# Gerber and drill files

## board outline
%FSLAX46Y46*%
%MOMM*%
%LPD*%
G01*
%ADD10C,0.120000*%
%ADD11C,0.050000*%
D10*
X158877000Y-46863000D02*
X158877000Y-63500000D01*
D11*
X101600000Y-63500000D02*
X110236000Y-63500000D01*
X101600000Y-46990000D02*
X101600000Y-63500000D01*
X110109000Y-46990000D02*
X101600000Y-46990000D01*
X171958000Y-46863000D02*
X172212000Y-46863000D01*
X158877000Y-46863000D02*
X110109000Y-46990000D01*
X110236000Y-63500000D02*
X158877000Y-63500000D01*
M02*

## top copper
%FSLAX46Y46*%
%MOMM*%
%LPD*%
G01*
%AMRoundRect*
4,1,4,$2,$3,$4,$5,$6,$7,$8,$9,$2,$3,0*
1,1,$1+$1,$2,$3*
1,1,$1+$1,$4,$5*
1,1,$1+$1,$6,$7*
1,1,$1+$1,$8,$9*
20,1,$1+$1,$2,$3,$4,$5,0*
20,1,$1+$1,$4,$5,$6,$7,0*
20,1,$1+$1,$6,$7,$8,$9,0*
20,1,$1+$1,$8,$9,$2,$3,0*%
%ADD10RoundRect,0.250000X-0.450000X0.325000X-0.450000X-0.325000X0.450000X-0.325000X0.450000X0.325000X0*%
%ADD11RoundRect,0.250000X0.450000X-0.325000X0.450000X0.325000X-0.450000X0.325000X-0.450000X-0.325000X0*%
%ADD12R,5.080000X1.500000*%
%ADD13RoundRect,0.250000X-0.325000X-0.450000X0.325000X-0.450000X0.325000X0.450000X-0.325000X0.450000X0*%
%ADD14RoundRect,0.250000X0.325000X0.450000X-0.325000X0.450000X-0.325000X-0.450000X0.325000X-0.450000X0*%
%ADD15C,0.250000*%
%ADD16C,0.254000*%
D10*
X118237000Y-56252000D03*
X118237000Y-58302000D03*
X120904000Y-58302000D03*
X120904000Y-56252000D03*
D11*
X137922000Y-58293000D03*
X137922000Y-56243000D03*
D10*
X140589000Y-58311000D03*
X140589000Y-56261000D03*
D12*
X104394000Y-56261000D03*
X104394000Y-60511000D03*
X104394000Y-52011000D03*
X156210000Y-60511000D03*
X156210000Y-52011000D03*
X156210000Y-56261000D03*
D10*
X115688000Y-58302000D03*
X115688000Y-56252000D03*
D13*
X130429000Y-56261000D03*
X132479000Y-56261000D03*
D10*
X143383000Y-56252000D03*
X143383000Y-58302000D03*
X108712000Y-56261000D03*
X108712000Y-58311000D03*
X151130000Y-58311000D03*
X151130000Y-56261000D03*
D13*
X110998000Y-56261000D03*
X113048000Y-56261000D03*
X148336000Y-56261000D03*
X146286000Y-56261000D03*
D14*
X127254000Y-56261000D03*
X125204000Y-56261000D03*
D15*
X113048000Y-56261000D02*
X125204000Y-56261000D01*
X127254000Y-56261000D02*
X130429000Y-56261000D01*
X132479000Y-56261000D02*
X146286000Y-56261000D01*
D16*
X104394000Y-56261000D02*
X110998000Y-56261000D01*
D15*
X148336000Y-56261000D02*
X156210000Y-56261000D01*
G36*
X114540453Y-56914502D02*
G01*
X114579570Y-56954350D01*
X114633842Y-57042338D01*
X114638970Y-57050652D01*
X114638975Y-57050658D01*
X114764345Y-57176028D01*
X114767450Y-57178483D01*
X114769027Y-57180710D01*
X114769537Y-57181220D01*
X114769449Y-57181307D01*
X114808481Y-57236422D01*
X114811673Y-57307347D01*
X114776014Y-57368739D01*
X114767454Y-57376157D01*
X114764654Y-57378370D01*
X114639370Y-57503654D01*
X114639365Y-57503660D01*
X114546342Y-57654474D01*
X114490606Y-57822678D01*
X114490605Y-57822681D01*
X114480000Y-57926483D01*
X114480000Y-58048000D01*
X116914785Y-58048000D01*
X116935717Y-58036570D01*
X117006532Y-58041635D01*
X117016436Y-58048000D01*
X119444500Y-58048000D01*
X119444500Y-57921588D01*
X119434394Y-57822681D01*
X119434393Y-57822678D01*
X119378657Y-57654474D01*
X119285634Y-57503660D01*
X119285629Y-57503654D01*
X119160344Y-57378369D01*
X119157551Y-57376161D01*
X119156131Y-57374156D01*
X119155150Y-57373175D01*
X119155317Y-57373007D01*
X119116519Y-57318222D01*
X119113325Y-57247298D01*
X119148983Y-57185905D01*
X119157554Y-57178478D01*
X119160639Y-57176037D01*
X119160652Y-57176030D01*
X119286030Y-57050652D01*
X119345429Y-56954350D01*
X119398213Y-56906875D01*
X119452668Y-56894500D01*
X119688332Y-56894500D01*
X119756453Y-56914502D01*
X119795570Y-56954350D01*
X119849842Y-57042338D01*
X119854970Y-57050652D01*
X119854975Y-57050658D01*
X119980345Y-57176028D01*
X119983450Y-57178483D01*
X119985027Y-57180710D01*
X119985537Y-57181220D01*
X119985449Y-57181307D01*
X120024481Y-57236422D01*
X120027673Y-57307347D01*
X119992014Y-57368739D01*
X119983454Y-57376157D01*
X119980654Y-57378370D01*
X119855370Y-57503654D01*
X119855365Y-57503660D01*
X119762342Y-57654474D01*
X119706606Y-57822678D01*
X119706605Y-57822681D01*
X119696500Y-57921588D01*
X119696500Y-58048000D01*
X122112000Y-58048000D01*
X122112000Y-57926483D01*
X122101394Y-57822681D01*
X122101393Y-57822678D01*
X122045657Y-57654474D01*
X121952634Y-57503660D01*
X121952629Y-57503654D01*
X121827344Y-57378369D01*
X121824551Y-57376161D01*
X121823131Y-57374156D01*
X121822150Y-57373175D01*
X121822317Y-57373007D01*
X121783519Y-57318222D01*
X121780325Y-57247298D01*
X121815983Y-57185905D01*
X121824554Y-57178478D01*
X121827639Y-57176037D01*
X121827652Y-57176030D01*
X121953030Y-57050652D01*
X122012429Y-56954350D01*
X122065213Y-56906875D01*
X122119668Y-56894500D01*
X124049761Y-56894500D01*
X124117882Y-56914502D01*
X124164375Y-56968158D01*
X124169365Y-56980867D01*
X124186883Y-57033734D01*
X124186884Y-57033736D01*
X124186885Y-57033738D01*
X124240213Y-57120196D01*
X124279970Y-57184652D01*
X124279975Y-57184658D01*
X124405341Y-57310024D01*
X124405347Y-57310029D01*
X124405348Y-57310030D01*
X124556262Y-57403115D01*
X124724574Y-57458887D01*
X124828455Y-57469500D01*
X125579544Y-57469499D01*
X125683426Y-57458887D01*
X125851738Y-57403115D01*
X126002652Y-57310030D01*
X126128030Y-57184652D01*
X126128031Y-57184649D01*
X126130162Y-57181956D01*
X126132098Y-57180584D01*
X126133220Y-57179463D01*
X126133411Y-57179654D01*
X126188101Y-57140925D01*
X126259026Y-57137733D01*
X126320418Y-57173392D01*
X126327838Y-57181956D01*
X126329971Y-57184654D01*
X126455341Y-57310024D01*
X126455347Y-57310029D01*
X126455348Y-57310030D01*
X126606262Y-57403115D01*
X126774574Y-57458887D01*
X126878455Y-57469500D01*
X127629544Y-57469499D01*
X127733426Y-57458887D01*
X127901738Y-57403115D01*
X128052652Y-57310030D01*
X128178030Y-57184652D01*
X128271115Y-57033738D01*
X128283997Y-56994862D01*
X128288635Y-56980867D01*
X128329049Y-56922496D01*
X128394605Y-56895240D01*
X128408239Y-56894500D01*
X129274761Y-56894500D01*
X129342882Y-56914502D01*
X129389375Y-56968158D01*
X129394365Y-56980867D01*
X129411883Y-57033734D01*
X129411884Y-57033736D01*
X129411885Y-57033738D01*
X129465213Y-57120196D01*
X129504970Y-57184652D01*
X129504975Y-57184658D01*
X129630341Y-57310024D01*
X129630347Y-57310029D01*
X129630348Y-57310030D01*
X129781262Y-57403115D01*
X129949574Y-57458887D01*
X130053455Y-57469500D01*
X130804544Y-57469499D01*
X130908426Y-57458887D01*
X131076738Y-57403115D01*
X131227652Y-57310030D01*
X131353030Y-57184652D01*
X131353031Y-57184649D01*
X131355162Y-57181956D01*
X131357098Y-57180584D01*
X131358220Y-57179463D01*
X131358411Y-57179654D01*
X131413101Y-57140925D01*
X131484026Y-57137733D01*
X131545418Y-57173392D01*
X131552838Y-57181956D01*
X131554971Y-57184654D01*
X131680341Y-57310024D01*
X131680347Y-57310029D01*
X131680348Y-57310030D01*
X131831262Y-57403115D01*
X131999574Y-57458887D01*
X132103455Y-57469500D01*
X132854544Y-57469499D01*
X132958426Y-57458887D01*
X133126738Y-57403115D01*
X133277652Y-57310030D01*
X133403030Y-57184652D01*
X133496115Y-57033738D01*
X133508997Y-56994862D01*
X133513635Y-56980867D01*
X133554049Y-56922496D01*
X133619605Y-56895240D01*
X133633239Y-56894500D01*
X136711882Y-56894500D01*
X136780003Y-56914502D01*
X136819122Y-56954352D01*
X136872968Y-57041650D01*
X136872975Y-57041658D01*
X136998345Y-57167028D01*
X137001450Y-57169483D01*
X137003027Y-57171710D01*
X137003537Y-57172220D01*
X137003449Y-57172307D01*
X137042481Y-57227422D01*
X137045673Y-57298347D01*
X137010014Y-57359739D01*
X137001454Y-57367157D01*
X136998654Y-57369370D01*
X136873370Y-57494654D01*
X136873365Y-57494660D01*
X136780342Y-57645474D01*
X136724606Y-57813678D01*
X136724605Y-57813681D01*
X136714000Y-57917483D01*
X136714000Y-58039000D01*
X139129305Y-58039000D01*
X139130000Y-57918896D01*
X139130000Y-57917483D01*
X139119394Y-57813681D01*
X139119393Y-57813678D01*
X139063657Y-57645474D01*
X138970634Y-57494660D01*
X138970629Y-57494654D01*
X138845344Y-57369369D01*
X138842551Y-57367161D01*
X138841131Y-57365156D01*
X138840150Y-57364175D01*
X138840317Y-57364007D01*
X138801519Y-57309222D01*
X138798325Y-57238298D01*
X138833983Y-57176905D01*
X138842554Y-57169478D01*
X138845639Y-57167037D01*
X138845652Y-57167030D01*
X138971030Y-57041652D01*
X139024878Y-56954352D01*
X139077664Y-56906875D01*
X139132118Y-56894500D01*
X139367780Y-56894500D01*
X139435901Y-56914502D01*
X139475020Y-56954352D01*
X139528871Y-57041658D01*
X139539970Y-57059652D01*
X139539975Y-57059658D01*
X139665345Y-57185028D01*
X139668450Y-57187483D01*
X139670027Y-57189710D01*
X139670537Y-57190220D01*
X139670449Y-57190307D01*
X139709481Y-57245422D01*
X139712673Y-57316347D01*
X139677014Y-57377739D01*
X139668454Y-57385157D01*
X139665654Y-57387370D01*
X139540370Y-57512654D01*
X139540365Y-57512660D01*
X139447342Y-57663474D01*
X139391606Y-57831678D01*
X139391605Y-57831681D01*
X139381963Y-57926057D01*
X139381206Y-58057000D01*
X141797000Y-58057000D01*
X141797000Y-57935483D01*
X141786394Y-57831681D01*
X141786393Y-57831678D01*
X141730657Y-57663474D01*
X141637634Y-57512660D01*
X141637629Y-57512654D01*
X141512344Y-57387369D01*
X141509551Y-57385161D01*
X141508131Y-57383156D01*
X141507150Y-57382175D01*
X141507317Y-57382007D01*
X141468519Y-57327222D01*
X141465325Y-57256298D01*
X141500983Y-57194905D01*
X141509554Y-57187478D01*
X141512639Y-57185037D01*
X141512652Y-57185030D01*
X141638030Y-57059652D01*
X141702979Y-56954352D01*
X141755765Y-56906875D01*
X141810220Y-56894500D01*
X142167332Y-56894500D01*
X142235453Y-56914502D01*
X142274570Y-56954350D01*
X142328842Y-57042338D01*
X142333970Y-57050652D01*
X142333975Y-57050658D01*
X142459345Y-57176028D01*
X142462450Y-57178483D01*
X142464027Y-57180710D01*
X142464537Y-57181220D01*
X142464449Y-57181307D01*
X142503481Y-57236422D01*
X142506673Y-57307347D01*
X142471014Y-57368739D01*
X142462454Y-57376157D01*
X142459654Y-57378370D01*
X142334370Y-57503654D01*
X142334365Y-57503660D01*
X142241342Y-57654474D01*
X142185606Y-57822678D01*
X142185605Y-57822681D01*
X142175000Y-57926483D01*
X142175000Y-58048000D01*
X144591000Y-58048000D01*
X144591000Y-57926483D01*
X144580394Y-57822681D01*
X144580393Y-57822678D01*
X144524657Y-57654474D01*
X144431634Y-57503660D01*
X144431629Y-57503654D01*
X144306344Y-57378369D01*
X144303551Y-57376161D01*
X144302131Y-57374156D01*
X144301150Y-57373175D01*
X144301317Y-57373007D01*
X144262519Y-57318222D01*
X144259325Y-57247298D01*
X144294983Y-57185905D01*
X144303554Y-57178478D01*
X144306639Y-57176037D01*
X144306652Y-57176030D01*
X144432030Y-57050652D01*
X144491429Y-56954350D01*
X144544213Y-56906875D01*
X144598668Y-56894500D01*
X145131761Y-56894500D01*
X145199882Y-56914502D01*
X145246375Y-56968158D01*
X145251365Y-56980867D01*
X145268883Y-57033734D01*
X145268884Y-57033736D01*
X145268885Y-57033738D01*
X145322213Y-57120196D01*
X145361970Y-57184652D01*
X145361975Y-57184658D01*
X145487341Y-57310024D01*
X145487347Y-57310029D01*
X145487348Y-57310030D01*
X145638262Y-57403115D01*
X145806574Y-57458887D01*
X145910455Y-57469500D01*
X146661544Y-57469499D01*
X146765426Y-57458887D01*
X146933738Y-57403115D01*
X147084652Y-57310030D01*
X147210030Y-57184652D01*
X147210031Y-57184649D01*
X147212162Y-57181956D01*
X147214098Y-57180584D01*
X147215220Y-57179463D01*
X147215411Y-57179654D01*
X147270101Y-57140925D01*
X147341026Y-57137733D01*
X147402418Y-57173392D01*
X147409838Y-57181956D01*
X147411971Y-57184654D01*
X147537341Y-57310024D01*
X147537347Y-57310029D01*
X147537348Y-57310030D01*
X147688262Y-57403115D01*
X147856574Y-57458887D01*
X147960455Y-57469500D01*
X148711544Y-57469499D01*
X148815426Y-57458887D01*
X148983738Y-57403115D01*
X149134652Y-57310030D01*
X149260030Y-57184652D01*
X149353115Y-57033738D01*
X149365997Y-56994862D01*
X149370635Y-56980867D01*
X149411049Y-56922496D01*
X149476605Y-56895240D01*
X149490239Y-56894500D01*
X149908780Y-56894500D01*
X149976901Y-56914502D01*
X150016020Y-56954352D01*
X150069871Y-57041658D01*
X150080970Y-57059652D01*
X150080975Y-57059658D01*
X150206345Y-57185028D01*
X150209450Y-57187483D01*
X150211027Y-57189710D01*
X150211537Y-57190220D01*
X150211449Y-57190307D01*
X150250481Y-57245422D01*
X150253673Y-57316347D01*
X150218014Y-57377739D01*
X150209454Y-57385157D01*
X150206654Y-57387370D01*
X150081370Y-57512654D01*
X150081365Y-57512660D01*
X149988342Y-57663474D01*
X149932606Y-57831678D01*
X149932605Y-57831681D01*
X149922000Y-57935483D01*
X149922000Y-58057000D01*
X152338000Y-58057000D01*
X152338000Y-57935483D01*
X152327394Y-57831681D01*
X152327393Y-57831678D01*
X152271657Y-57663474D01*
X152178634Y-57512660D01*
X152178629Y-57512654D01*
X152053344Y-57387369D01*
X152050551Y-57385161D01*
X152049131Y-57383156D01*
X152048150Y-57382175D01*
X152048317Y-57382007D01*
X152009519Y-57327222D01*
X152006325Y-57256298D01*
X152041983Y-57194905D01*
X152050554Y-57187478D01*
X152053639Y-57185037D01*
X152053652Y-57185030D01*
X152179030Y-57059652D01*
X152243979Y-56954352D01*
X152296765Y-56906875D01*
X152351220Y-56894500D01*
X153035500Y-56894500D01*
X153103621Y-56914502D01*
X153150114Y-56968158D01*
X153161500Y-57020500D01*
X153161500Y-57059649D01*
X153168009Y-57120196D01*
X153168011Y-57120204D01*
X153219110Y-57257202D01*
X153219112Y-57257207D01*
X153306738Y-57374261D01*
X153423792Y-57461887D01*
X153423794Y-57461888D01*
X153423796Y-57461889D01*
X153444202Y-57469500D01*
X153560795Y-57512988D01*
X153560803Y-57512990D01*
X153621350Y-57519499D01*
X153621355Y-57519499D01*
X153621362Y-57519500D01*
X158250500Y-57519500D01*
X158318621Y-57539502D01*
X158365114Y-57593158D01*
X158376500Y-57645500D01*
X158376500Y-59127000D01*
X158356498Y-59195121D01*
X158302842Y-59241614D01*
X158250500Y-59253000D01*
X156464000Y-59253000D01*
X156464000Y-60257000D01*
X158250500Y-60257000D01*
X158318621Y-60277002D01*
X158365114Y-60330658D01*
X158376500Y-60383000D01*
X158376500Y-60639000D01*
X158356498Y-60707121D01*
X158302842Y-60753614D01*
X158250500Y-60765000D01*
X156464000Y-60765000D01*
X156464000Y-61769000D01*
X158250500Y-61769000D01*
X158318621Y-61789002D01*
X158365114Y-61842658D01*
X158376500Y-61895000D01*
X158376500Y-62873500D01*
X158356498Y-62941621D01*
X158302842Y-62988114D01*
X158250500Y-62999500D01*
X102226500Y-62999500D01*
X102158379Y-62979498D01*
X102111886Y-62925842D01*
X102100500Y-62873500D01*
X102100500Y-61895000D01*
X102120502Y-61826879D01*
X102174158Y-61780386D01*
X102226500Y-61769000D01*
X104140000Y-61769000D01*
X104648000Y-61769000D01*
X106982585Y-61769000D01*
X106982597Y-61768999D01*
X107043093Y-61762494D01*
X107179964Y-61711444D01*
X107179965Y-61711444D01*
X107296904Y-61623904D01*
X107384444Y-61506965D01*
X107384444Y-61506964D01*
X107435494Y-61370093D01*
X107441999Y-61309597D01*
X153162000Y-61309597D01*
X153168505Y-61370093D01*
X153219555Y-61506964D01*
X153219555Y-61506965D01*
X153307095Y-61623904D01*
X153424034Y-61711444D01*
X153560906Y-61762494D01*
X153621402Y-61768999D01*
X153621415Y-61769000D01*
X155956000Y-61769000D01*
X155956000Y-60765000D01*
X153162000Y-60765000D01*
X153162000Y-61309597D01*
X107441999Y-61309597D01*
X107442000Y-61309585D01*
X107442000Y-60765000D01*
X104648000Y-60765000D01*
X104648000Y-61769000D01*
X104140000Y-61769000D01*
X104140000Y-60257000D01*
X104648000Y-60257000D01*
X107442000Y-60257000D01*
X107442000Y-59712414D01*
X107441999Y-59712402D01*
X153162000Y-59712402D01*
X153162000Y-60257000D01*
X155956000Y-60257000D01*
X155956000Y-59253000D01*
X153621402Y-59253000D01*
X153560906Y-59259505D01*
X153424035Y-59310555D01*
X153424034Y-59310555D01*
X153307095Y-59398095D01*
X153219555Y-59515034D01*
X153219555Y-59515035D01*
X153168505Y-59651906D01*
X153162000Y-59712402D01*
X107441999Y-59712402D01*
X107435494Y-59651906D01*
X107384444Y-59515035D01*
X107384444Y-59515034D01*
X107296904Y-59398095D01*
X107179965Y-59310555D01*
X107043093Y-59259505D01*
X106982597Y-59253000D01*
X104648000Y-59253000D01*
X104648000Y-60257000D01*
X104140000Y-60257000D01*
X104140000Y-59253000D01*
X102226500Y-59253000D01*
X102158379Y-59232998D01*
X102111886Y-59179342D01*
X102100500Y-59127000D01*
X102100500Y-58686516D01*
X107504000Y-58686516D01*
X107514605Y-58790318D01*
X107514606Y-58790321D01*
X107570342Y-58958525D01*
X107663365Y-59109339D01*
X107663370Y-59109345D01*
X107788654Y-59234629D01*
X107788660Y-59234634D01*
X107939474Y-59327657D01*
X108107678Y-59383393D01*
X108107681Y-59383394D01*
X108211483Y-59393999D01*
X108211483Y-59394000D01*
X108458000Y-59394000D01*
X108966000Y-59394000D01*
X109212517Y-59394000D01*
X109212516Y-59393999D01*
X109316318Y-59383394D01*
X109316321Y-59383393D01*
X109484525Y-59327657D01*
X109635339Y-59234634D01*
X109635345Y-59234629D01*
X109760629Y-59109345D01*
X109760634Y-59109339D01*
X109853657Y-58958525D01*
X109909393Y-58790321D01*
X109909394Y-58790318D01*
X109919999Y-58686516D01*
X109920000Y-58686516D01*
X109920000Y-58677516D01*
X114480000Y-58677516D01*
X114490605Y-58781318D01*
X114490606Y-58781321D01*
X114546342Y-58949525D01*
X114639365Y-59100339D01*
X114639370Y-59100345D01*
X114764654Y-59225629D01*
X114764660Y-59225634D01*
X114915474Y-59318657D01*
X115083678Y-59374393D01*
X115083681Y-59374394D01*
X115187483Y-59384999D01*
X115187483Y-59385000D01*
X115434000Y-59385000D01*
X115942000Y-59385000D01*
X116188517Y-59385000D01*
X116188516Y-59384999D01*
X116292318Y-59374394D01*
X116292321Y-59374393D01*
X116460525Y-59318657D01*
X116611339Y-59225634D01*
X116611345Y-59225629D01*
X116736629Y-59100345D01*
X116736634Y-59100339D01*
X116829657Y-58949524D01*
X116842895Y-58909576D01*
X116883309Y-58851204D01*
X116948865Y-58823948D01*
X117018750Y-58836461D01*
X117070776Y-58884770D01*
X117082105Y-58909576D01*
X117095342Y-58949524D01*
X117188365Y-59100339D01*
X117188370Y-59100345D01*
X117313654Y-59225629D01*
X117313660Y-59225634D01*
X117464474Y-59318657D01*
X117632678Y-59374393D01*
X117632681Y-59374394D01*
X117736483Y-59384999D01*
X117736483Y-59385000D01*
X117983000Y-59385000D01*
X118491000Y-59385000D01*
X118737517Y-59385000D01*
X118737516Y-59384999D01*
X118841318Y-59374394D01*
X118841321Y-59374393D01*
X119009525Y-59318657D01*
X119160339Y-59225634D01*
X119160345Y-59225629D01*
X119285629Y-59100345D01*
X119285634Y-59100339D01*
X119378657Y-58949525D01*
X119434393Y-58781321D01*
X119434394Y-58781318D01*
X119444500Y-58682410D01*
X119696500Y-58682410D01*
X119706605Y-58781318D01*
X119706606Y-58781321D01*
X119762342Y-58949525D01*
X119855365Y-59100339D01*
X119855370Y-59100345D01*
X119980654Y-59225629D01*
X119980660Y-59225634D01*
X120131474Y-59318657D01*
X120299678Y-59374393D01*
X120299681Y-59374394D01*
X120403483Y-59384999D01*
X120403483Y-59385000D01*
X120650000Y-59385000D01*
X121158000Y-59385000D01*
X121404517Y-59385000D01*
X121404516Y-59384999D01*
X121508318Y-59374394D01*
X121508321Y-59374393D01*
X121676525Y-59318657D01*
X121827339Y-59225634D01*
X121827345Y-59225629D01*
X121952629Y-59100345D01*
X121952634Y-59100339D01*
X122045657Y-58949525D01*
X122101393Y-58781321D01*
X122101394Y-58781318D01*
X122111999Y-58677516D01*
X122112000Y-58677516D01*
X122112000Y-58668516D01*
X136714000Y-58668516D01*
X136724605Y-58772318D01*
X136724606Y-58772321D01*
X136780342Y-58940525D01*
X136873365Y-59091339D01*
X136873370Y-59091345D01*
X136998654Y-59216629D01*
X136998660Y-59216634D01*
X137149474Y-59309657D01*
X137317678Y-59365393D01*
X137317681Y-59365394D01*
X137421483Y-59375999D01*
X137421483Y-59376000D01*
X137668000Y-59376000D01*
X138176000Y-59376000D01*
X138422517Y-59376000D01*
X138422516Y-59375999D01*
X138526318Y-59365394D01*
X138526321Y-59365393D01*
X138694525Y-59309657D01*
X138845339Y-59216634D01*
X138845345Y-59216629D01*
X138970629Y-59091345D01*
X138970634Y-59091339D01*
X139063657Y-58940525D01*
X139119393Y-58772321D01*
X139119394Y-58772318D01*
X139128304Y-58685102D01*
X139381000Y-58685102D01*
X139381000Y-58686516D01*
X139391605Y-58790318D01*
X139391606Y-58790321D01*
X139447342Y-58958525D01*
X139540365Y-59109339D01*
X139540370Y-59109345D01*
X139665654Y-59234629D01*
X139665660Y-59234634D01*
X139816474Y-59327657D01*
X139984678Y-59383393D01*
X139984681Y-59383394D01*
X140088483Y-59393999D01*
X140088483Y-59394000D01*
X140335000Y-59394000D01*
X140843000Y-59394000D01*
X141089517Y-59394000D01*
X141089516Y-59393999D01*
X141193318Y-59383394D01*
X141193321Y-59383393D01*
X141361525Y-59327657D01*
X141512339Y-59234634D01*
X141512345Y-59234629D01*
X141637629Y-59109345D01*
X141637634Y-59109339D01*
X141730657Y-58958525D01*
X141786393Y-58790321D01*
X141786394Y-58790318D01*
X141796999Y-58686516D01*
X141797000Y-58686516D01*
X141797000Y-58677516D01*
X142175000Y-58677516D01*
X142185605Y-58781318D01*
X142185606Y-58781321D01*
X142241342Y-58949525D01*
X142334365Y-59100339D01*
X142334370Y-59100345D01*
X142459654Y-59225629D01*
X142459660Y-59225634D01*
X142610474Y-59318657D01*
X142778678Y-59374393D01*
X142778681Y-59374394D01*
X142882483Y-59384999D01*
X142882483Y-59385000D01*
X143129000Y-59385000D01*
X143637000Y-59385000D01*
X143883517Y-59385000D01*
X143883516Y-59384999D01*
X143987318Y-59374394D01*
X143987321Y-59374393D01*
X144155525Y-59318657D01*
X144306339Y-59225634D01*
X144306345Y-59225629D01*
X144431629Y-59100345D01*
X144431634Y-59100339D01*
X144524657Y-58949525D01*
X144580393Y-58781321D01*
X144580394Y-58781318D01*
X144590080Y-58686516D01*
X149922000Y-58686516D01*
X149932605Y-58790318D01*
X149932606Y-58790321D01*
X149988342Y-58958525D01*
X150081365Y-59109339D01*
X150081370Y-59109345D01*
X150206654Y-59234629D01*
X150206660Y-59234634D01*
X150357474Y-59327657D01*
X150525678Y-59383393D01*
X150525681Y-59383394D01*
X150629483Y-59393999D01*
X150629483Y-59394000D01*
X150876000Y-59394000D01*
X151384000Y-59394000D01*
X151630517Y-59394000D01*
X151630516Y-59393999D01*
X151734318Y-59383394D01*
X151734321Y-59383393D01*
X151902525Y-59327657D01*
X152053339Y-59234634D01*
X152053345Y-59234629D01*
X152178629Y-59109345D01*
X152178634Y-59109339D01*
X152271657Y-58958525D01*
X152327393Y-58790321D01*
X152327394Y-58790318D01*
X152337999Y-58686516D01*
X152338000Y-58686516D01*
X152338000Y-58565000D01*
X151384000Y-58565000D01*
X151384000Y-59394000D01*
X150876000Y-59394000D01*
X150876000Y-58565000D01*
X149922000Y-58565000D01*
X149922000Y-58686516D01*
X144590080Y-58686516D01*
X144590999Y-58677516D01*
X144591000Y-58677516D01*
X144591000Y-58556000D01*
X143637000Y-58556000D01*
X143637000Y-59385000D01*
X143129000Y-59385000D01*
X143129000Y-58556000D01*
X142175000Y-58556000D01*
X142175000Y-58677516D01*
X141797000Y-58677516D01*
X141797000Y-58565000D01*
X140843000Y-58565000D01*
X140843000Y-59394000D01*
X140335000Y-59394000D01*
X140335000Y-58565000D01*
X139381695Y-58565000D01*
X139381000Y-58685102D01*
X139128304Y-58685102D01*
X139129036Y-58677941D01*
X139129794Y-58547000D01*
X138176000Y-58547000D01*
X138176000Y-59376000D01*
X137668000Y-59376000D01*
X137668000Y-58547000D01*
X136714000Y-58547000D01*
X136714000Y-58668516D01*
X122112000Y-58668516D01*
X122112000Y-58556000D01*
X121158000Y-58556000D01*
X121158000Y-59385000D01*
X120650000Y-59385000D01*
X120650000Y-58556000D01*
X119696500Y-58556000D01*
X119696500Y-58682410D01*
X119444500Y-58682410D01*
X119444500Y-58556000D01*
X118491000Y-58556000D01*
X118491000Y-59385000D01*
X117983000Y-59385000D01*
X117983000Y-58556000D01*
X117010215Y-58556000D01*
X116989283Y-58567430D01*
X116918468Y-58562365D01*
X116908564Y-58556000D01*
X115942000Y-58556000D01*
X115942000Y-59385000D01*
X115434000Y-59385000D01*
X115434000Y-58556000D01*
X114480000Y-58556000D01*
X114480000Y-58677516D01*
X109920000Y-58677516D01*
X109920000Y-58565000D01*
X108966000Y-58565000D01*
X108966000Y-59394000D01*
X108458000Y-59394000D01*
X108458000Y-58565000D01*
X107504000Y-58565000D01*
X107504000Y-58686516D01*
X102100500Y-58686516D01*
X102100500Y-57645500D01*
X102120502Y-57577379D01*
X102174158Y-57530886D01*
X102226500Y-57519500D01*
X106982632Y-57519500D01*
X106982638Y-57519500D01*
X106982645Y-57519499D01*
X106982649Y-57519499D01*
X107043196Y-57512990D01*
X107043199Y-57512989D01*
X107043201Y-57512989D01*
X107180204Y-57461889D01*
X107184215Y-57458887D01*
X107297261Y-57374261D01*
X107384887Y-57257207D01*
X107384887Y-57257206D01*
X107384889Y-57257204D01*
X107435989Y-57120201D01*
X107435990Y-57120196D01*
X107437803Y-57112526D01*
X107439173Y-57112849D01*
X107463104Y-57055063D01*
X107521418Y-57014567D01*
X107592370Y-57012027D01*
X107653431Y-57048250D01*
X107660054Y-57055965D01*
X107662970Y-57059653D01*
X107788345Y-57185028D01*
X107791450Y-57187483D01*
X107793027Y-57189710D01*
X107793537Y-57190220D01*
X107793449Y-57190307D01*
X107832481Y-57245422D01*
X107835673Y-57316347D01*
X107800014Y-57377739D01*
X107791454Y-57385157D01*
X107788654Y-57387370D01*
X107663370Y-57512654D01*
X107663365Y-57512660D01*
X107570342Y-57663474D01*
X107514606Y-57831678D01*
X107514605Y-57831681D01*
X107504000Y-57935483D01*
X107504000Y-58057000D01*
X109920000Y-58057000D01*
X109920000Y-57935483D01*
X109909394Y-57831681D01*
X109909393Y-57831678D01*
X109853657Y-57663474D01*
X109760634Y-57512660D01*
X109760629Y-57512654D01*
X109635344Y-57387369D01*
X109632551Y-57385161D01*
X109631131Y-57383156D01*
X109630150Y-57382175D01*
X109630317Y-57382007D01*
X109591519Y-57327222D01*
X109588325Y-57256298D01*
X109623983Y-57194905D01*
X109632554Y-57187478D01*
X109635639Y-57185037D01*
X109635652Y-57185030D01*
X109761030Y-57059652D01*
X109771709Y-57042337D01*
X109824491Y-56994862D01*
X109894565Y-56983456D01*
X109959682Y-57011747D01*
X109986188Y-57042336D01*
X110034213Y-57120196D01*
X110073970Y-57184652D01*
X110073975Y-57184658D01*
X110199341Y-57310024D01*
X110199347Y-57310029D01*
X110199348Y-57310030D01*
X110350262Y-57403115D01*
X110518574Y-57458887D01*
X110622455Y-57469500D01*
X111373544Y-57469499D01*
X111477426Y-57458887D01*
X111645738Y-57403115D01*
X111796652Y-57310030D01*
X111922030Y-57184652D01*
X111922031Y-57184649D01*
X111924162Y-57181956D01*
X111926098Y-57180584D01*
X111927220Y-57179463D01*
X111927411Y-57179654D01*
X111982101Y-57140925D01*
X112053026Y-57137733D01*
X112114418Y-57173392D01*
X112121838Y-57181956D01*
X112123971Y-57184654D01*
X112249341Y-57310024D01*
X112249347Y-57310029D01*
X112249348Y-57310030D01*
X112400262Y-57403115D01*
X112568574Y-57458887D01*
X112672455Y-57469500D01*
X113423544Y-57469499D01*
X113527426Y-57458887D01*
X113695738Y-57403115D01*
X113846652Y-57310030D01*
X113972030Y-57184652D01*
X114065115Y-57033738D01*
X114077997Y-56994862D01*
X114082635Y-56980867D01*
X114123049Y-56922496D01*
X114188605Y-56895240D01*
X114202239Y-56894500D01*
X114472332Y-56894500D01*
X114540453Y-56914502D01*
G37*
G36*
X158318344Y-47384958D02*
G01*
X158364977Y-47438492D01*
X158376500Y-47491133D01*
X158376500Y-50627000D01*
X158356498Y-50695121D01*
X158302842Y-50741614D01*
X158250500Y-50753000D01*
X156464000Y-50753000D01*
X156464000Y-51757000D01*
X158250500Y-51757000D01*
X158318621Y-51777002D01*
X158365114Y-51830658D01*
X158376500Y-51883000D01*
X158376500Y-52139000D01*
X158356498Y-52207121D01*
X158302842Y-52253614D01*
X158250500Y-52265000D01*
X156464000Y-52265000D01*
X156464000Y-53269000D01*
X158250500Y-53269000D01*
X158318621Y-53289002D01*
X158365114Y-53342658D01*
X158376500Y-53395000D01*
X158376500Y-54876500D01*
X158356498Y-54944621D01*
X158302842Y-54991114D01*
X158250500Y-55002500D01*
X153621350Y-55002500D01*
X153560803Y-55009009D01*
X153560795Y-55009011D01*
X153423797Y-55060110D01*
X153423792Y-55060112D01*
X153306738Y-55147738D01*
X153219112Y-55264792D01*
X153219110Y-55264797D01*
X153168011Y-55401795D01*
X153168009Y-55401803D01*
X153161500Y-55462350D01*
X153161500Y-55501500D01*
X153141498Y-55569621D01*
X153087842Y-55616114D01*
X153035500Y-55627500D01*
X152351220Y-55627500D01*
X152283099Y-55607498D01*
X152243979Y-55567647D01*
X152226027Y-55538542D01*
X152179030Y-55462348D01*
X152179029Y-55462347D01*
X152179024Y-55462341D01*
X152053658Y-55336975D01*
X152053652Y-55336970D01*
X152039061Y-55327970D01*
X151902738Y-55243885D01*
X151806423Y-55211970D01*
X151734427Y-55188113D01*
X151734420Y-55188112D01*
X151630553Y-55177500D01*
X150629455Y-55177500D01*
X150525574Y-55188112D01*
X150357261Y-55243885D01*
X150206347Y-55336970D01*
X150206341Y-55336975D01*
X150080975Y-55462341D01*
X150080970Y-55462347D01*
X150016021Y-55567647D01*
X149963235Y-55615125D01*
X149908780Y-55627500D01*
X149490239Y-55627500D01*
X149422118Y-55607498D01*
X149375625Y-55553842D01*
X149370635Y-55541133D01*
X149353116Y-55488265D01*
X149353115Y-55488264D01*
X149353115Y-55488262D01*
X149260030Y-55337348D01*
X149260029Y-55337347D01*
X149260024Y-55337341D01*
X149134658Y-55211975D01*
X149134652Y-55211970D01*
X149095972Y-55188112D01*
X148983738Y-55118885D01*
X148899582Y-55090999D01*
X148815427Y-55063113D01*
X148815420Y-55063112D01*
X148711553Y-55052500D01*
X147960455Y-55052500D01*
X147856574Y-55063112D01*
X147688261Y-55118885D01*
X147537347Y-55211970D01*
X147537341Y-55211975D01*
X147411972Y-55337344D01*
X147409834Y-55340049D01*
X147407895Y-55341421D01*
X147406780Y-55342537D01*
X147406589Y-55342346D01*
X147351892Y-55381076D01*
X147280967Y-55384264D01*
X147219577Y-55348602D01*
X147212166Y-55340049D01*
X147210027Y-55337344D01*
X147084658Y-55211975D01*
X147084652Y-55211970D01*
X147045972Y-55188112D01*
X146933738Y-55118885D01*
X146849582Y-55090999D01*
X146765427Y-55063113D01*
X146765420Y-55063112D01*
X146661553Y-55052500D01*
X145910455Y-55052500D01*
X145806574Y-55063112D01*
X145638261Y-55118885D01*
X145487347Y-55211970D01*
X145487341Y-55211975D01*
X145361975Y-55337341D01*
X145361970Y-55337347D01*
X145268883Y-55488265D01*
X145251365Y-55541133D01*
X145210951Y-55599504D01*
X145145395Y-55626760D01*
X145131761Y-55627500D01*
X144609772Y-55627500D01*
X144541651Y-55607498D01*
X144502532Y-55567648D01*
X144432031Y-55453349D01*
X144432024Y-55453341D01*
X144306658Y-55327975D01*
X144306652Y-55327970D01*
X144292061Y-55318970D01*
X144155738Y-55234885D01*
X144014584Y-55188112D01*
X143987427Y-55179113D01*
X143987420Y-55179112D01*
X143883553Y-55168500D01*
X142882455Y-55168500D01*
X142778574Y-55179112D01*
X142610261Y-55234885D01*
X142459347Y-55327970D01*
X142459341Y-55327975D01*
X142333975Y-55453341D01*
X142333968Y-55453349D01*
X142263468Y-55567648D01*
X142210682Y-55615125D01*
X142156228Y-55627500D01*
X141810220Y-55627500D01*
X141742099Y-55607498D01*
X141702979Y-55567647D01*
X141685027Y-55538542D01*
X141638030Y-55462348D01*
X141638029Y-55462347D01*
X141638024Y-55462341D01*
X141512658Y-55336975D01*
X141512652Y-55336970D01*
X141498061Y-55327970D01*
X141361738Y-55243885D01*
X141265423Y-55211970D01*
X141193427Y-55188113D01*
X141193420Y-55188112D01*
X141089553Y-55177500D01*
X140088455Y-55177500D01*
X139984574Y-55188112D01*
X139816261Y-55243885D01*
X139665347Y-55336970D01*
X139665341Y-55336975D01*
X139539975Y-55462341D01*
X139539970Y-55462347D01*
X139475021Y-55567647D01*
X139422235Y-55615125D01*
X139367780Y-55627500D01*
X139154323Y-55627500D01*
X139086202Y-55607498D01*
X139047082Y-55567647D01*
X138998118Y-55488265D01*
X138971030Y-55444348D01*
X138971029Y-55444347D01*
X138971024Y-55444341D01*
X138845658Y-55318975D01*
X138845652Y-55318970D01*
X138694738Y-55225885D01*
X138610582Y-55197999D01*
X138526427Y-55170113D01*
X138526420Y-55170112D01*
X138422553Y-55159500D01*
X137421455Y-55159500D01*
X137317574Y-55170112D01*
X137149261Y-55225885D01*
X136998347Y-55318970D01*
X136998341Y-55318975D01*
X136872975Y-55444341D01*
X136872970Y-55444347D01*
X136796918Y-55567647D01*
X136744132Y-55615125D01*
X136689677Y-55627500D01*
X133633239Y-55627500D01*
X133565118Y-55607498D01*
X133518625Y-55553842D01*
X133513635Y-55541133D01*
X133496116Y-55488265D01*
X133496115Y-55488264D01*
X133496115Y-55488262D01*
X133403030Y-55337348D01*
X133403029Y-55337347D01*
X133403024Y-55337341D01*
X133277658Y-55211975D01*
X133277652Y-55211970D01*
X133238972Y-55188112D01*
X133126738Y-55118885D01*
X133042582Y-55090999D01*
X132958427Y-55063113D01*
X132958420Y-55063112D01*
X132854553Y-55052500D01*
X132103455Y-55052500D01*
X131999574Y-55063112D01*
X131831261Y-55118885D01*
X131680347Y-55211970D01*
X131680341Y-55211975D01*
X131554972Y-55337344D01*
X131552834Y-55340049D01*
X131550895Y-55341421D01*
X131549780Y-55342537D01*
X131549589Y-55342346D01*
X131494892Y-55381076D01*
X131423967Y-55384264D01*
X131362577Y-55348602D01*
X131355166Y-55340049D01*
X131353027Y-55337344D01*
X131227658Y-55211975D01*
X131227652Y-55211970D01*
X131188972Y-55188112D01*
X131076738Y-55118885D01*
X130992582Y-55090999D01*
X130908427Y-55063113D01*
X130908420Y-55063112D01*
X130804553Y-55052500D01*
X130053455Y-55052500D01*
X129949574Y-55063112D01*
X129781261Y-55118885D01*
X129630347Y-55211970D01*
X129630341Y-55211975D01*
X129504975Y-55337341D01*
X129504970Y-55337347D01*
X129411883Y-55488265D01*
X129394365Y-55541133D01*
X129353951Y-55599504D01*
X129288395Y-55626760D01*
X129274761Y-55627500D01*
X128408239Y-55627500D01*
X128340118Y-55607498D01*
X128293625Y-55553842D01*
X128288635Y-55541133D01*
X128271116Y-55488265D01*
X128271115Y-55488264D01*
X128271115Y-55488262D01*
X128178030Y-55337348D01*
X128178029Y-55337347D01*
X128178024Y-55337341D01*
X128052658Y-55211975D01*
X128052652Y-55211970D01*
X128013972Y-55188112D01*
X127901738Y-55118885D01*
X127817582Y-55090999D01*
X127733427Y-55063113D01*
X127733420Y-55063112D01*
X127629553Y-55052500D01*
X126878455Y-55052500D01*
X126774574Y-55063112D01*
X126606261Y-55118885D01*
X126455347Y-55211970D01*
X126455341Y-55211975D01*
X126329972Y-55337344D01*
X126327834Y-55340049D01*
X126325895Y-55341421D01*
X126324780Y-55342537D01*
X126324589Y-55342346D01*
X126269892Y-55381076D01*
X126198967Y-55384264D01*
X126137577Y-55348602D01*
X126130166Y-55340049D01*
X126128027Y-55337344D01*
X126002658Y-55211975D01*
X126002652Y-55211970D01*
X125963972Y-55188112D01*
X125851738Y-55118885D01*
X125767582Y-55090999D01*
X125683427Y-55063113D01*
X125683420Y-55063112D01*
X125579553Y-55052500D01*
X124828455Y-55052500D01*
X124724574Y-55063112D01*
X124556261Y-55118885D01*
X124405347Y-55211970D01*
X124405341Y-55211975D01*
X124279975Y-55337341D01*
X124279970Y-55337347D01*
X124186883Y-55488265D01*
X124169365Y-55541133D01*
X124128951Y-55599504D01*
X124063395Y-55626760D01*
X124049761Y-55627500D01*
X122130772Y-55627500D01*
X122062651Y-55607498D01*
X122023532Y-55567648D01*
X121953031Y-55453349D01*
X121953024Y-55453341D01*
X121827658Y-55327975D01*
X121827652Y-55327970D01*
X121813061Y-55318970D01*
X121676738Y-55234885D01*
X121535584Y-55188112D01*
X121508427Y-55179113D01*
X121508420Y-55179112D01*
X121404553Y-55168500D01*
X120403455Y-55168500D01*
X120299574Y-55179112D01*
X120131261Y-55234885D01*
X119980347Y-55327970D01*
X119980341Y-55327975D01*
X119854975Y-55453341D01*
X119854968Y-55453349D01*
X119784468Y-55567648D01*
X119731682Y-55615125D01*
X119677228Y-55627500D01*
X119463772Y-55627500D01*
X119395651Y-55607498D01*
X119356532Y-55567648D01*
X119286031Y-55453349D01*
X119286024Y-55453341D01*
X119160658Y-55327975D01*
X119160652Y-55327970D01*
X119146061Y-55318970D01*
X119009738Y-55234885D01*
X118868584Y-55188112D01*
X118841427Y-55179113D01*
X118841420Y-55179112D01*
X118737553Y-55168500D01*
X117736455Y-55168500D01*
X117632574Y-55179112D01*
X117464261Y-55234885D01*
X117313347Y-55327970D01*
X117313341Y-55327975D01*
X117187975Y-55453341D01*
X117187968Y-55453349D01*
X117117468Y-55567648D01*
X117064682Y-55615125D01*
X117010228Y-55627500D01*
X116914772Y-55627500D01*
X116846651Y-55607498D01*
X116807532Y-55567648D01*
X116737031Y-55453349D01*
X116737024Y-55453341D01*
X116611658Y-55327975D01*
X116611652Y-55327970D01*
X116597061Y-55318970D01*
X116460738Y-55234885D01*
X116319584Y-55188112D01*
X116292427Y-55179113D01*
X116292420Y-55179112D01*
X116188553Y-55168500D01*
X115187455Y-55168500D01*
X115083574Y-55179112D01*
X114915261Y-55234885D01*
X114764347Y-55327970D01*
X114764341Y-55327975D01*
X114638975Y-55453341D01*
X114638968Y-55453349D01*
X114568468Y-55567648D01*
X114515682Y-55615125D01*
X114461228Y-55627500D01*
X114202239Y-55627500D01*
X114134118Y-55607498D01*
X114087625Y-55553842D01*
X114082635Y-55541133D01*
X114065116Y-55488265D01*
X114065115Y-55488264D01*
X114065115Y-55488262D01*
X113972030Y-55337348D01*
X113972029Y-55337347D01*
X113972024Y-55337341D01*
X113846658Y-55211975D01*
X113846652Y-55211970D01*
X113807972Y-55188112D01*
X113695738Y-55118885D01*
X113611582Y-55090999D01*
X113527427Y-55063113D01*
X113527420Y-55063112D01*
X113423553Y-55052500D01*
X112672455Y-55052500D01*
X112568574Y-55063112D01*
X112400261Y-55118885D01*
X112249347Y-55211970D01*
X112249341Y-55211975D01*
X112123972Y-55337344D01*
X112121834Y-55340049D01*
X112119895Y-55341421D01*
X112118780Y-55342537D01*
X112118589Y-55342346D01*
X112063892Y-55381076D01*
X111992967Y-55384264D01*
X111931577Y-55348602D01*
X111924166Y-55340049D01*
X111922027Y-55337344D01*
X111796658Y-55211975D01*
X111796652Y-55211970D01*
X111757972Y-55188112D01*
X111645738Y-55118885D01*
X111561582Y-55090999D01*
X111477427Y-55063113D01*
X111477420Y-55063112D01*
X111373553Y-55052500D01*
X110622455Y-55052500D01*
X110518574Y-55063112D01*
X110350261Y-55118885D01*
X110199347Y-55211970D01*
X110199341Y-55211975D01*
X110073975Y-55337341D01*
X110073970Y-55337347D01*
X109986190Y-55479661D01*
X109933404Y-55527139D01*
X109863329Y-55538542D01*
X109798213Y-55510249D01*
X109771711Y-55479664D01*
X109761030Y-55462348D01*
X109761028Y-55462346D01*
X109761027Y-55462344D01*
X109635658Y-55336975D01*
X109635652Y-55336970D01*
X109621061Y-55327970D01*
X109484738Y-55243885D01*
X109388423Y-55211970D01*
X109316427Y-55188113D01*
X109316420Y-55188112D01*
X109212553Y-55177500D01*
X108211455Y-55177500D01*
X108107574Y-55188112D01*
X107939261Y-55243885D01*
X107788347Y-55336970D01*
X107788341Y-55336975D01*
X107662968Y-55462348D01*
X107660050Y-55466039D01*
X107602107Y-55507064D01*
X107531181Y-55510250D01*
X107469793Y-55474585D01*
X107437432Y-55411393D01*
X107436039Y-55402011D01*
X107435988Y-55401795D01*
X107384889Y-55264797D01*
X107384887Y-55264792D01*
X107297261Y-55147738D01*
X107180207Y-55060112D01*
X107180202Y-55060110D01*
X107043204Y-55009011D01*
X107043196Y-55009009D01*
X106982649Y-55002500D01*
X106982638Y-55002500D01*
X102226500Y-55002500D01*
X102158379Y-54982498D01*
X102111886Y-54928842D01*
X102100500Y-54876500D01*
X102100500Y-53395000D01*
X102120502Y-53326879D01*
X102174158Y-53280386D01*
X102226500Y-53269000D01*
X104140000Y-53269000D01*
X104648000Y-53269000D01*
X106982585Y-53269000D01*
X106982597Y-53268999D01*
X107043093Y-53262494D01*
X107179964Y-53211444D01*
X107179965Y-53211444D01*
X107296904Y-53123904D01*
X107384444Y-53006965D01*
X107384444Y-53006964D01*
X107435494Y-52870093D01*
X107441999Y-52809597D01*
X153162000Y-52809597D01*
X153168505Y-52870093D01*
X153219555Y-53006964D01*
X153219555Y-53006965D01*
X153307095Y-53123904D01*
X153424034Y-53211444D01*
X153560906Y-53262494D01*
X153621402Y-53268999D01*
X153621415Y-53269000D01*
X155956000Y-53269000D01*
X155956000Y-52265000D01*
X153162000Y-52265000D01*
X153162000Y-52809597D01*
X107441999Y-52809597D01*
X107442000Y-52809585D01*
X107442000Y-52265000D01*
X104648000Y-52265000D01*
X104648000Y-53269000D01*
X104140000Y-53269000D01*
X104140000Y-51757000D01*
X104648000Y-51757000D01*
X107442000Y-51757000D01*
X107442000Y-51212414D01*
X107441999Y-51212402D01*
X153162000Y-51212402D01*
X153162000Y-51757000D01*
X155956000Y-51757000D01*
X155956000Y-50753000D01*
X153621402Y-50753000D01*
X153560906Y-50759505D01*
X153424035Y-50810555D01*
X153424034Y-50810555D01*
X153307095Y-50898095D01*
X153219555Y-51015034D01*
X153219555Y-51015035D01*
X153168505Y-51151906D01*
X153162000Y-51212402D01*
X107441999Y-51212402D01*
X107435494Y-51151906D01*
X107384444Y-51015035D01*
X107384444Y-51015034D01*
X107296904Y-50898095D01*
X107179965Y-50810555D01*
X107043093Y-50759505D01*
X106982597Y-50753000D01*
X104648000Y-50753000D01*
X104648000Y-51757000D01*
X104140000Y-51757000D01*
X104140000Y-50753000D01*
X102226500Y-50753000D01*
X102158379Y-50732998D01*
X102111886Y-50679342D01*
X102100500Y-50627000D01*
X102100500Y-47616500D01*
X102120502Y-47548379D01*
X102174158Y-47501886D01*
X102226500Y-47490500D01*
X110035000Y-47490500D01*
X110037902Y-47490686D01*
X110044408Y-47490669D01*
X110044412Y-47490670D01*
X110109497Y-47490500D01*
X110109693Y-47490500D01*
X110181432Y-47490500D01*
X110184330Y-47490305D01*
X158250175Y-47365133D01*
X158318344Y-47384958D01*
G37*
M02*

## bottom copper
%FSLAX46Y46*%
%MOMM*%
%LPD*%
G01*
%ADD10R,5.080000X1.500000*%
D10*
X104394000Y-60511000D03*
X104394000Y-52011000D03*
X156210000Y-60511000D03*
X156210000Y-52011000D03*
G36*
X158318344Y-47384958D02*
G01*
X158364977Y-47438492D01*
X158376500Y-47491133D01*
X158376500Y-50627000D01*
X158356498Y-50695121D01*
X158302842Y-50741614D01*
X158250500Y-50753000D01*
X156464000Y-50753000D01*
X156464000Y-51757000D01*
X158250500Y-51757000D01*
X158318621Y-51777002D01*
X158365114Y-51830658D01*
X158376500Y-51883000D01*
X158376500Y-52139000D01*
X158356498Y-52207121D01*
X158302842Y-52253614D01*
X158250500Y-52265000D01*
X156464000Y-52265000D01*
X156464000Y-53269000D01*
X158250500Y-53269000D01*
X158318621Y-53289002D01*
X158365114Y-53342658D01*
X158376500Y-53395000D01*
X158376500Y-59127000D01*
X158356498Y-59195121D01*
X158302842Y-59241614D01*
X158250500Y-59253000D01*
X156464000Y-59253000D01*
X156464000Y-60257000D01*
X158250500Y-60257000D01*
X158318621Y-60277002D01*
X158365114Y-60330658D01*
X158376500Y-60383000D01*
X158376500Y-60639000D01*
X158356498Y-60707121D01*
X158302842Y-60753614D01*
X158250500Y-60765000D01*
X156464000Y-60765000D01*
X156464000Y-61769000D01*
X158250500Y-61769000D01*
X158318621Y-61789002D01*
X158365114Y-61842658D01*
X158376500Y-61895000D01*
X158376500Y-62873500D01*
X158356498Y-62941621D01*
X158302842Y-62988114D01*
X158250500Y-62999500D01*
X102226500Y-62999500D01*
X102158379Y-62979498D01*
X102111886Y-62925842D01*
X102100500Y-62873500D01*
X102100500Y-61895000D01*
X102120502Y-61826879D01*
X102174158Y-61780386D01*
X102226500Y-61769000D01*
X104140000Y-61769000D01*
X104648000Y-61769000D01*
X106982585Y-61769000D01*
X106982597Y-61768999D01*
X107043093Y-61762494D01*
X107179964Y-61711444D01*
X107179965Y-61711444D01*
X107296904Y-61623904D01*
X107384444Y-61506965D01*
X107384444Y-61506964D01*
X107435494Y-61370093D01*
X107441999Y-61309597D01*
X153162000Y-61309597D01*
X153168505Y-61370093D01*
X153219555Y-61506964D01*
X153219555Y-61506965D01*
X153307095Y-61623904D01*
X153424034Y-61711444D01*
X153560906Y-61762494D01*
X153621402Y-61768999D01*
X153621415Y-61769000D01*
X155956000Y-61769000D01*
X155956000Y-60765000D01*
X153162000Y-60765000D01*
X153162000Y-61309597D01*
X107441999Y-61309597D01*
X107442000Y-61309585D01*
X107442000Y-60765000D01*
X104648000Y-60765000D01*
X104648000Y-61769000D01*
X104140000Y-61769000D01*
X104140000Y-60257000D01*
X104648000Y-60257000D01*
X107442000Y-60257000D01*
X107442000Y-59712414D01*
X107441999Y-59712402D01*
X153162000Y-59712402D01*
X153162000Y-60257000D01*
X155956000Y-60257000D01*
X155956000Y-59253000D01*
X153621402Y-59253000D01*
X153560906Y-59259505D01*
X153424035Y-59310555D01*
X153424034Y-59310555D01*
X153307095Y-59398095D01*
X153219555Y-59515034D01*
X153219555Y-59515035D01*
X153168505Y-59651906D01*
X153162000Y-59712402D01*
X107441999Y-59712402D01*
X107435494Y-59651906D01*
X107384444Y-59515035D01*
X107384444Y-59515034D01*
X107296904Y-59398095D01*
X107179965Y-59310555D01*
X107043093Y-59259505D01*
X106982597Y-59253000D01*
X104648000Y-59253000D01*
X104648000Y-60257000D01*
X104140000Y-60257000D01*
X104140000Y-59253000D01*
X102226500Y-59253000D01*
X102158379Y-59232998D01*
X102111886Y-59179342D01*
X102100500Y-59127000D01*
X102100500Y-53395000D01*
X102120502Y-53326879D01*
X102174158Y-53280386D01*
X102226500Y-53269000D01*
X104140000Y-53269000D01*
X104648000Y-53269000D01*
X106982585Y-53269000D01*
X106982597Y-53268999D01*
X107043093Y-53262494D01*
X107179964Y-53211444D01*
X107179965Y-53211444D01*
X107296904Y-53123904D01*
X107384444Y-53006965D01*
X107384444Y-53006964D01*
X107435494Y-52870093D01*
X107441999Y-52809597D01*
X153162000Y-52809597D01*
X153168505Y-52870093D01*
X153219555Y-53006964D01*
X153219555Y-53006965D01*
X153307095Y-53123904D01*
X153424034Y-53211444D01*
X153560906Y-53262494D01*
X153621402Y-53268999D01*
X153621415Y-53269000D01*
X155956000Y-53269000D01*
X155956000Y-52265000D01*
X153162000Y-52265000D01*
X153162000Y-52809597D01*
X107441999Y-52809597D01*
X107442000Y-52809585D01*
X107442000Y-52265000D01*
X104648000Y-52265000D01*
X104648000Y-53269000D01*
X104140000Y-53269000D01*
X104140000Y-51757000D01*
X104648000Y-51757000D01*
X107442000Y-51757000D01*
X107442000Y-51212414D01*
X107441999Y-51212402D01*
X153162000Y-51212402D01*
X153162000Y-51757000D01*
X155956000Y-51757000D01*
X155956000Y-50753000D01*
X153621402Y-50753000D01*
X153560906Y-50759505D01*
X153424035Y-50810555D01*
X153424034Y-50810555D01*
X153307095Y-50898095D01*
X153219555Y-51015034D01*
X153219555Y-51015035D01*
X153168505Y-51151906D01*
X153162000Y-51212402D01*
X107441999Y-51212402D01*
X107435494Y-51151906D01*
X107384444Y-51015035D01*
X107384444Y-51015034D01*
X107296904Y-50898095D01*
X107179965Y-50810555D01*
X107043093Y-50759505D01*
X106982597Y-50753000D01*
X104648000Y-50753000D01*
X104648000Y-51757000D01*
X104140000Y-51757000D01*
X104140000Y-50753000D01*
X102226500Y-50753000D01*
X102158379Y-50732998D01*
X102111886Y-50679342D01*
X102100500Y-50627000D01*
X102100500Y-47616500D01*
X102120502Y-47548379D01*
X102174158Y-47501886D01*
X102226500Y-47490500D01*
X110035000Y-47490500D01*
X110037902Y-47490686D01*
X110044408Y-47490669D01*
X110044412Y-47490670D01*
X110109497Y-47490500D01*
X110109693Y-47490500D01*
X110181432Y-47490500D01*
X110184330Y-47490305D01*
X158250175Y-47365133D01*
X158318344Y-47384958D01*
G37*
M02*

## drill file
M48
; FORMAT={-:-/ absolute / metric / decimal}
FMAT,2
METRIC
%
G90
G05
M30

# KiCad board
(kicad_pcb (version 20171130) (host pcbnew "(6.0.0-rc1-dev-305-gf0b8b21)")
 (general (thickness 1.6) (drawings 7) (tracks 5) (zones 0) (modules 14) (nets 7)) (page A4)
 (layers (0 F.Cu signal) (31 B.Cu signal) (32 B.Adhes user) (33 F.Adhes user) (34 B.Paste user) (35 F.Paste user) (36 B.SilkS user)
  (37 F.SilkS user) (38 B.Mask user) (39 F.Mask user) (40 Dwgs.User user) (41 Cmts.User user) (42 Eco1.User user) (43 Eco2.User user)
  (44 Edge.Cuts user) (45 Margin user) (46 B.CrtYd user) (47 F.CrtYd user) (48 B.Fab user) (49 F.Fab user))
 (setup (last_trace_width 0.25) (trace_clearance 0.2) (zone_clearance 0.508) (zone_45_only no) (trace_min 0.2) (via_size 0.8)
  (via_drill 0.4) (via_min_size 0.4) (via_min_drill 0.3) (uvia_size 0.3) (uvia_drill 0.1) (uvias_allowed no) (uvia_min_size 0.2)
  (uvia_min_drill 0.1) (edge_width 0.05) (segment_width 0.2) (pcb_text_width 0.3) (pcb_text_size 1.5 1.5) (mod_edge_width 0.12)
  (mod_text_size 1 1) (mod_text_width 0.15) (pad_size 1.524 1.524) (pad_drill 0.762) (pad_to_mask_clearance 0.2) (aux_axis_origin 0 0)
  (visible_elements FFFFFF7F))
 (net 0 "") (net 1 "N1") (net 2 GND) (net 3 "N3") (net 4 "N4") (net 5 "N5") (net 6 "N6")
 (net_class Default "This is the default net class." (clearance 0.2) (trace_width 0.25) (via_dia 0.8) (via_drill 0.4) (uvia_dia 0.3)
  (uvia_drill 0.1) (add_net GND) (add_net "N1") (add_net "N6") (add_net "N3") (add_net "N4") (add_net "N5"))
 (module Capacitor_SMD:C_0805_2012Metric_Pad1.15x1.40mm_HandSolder (layer F.Cu) (at 118.237 57.277 270)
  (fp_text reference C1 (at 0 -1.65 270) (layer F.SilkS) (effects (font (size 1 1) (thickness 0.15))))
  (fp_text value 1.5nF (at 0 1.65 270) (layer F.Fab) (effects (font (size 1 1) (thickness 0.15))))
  (pad 1 smd roundrect (at -1.025 0 270) (size 1.15 1.4) (layers F.Cu F.Paste F.Mask) (roundrect_rratio 0.217391) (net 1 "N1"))
  (pad 2 smd roundrect (at 1.025 0 270) (size 1.15 1.4) (layers F.Cu F.Paste F.Mask) (roundrect_rratio 0.217391) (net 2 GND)))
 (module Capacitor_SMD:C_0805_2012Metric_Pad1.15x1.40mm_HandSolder (layer F.Cu) (at 120.904 57.277 270)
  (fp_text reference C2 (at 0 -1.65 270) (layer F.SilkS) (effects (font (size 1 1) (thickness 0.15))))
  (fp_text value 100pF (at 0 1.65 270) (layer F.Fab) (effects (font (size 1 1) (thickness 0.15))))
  (pad 2 smd roundrect (at 1.025 0 270) (size 1.15 1.4) (layers F.Cu F.Paste F.Mask) (roundrect_rratio 0.217391) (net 2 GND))
  (pad 1 smd roundrect (at -1.025 0 270) (size 1.15 1.4) (layers F.Cu F.Paste F.Mask) (roundrect_rratio 0.217391) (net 1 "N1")))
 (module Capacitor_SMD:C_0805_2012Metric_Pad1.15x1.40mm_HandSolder (layer F.Cu) (at 137.922 57.268 90)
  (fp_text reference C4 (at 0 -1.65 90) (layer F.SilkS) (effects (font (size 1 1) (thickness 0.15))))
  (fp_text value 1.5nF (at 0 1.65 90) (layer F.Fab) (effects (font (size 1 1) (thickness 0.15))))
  (pad 1 smd roundrect (at -1.025 0 90) (size 1.15 1.4) (layers F.Cu F.Paste F.Mask) (roundrect_rratio 0.217391) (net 2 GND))
  (pad 2 smd roundrect (at 1.025 0 90) (size 1.15 1.4) (layers F.Cu F.Paste F.Mask) (roundrect_rratio 0.217391) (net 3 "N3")))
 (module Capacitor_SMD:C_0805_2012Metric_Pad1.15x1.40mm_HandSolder (layer F.Cu) (at 140.589 57.286 270)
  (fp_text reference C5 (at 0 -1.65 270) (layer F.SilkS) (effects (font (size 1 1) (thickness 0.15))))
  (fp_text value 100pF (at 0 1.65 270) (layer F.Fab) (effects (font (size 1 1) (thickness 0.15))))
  (pad 2 smd roundrect (at 1.025 0 270) (size 1.15 1.4) (layers F.Cu F.Paste F.Mask) (roundrect_rratio 0.217391) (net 2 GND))
  (pad 1 smd roundrect (at -1.025 0 270) (size 1.15 1.4) (layers F.Cu F.Paste F.Mask) (roundrect_rratio 0.217391) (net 3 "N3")))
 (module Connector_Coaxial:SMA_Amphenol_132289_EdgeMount (layer F.Cu) (at 104.394 56.261 180)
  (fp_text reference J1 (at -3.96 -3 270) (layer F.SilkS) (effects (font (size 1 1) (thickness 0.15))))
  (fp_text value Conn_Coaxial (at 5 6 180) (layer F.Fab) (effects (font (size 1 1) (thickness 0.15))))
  (pad 1 smd rect (at 0 0 270) (size 1.5 5.08) (layers F.Cu F.Paste F.Mask) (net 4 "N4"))
  (pad 2 smd rect (at 0 -4.25 270) (size 1.5 5.08) (layers F.Cu F.Paste F.Mask) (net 2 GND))
  (pad 2 smd rect (at 0 4.25 270) (size 1.5 5.08) (layers F.Cu F.Paste F.Mask) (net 2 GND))
  (pad 2 smd rect (at 0 -4.25 270) (size 1.5 5.08) (layers B.Cu B.Paste B.Mask) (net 2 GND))
  (pad 2 smd rect (at 0 4.25 270) (size 1.5 5.08) (layers B.Cu B.Paste B.Mask) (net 2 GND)))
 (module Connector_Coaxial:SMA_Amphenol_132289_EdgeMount (layer F.Cu) (at 156.21 56.261)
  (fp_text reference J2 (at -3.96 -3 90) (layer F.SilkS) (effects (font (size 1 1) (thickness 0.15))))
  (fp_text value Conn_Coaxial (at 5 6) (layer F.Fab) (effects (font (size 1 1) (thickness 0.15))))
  (pad 2 smd rect (at 0 4.25 90) (size 1.5 5.08) (layers B.Cu B.Paste B.Mask) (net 2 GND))
  (pad 2 smd rect (at 0 -4.25 90) (size 1.5 5.08) (layers B.Cu B.Paste B.Mask) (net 2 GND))
  (pad 2 smd rect (at 0 4.25 90) (size 1.5 5.08) (layers F.Cu F.Paste F.Mask) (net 2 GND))
  (pad 2 smd rect (at 0 -4.25 90) (size 1.5 5.08) (layers F.Cu F.Paste F.Mask) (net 2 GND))
  (pad 1 smd rect (at 0 0 90) (size 1.5 5.08) (layers F.Cu F.Paste F.Mask) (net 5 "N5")))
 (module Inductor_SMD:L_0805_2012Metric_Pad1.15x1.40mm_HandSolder (layer F.Cu) (at 115.688 57.277 270)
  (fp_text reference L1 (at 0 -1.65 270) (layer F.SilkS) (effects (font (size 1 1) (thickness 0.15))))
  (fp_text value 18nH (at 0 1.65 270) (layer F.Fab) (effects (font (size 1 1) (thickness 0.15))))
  (pad 2 smd roundrect (at 1.025 0 270) (size 1.15 1.4) (layers F.Cu F.Paste F.Mask) (roundrect_rratio 0.217391) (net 2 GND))
  (pad 1 smd roundrect (at -1.025 0 270) (size 1.15 1.4) (layers F.Cu F.Paste F.Mask) (roundrect_rratio 0.217391) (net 1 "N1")))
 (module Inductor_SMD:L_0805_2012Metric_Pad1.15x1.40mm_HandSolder (layer F.Cu) (at 131.454 56.261)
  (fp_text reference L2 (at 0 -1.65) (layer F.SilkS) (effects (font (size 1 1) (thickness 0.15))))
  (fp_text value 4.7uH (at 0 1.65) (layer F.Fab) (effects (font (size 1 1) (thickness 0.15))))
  (pad 1 smd roundrect (at -1.025 0) (size 1.15 1.4) (layers F.Cu F.Paste F.Mask) (roundrect_rratio 0.217391) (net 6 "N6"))
  (pad 2 smd roundrect (at 1.025 0) (size 1.15 1.4) (layers F.Cu F.Paste F.Mask) (roundrect_rratio 0.217391) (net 3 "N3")))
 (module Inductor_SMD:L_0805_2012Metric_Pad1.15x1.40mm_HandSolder (layer F.Cu) (at 143.383 57.277 270)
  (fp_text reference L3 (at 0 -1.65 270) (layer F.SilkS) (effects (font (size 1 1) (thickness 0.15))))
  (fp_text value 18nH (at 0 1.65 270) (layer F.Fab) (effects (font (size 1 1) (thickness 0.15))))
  (pad 1 smd roundrect (at -1.025 0 270) (size 1.15 1.4) (layers F.Cu F.Paste F.Mask) (roundrect_rratio 0.217391) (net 3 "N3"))
  (pad 2 smd roundrect (at 1.025 0 270) (size 1.15 1.4) (layers F.Cu F.Paste F.Mask) (roundrect_rratio 0.217391) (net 2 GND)))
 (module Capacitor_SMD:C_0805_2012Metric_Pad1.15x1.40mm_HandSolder (layer F.Cu) (at 108.712 57.286 270)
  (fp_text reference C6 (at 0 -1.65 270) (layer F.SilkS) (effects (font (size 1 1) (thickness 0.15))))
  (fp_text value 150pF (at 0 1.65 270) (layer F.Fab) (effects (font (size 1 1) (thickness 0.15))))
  (pad 1 smd roundrect (at -1.025 0 270) (size 1.15 1.4) (layers F.Cu F.Paste F.Mask) (roundrect_rratio 0.217391) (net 4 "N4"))
  (pad 2 smd roundrect (at 1.025 0 270) (size 1.15 1.4) (layers F.Cu F.Paste F.Mask) (roundrect_rratio 0.217391) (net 2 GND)))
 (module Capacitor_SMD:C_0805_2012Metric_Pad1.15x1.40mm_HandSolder (layer F.Cu) (at 151.13 57.286 270)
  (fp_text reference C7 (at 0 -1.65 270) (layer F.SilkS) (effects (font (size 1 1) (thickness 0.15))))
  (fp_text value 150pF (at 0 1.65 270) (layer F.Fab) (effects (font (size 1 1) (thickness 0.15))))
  (pad 2 smd roundrect (at 1.025 0 270) (size 1.15 1.4) (layers F.Cu F.Paste F.Mask) (roundrect_rratio 0.217391) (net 2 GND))
  (pad 1 smd roundrect (at -1.025 0 270) (size 1.15 1.4) (layers F.Cu F.Paste F.Mask) (roundrect_rratio 0.217391) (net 5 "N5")))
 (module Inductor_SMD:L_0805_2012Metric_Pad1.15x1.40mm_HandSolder (layer F.Cu) (at 112.023 56.261)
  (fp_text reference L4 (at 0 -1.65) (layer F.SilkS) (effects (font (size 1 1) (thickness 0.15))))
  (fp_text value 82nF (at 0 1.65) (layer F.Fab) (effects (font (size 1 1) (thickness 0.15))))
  (pad 1 smd roundrect (at -1.025 0) (size 1.15 1.4) (layers F.Cu F.Paste F.Mask) (roundrect_rratio 0.217391) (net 4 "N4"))
  (pad 2 smd roundrect (at 1.025 0) (size 1.15 1.4) (layers F.Cu F.Paste F.Mask) (roundrect_rratio 0.217391) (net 1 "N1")))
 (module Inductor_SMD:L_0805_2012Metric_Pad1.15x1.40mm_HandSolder (layer F.Cu) (at 147.311 56.261)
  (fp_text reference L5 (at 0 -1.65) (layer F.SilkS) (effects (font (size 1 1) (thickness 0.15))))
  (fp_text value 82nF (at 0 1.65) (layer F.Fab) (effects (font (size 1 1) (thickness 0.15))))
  (pad 2 smd roundrect (at 1.025 0) (size 1.15 1.4) (layers F.Cu F.Paste F.Mask) (roundrect_rratio 0.217391) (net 5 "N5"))
  (pad 1 smd roundrect (at -1.025 0) (size 1.15 1.4) (layers F.Cu F.Paste F.Mask) (roundrect_rratio 0.217391) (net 3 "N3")))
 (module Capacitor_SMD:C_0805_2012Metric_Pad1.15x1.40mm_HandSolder (layer F.Cu) (at 126.229 56.261 180)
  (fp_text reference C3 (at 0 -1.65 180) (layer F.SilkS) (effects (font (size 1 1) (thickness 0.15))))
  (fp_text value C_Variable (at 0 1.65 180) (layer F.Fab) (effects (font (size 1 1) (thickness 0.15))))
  (pad 1 smd roundrect (at -1.025 0 180) (size 1.15 1.4) (layers F.Cu F.Paste F.Mask) (roundrect_rratio 0.217391) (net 6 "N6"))
  (pad 2 smd roundrect (at 1.025 0 180) (size 1.15 1.4) (layers F.Cu F.Paste F.Mask) (roundrect_rratio 0.217391) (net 1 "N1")))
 (gr_line (start 158.877 46.863) (end 158.877 63.5) (layer Edge.Cuts) (width 0.12))
 (gr_line (start 101.6 63.5) (end 110.236 63.5) (layer Edge.Cuts) (width 0.05))
 (gr_line (start 101.6 46.99) (end 101.6 63.5) (layer Edge.Cuts) (width 0.05))
 (gr_line (start 110.109 46.99) (end 101.6 46.99) (layer Edge.Cuts) (width 0.05))
 (gr_line (start 171.958 46.863) (end 172.212 46.863) (layer Edge.Cuts) (width 0.05))
 (gr_line (start 158.877 46.863) (end 110.109 46.99) (layer Edge.Cuts) (width 0.05))
 (gr_line (start 110.236 63.5) (end 158.877 63.5) (layer Edge.Cuts) (width 0.05))
 (segment (start 113.048 56.261) (end 125.204 56.261) (width 0.25) (layer F.Cu) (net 1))
 (segment (start 127.254 56.261) (end 130.429 56.261) (width 0.25) (layer F.Cu) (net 6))
 (segment (start 132.479 56.261) (end 146.286 56.261) (width 0.25) (layer F.Cu) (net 3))
 (segment (start 104.394 56.261) (end 110.998 56.261) (width 0.254) (layer F.Cu) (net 4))
 (segment (start 148.336 56.261) (end 156.21 56.261) (width 0.25) (layer F.Cu) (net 5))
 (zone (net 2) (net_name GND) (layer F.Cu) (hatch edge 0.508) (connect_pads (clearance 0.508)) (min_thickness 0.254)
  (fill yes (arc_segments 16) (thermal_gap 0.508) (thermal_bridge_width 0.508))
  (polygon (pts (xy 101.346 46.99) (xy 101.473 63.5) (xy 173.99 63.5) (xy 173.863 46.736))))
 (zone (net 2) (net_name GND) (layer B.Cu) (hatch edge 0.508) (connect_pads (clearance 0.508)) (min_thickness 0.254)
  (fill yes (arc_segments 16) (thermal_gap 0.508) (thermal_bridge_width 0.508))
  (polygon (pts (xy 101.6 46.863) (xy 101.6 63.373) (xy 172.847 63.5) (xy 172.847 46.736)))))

